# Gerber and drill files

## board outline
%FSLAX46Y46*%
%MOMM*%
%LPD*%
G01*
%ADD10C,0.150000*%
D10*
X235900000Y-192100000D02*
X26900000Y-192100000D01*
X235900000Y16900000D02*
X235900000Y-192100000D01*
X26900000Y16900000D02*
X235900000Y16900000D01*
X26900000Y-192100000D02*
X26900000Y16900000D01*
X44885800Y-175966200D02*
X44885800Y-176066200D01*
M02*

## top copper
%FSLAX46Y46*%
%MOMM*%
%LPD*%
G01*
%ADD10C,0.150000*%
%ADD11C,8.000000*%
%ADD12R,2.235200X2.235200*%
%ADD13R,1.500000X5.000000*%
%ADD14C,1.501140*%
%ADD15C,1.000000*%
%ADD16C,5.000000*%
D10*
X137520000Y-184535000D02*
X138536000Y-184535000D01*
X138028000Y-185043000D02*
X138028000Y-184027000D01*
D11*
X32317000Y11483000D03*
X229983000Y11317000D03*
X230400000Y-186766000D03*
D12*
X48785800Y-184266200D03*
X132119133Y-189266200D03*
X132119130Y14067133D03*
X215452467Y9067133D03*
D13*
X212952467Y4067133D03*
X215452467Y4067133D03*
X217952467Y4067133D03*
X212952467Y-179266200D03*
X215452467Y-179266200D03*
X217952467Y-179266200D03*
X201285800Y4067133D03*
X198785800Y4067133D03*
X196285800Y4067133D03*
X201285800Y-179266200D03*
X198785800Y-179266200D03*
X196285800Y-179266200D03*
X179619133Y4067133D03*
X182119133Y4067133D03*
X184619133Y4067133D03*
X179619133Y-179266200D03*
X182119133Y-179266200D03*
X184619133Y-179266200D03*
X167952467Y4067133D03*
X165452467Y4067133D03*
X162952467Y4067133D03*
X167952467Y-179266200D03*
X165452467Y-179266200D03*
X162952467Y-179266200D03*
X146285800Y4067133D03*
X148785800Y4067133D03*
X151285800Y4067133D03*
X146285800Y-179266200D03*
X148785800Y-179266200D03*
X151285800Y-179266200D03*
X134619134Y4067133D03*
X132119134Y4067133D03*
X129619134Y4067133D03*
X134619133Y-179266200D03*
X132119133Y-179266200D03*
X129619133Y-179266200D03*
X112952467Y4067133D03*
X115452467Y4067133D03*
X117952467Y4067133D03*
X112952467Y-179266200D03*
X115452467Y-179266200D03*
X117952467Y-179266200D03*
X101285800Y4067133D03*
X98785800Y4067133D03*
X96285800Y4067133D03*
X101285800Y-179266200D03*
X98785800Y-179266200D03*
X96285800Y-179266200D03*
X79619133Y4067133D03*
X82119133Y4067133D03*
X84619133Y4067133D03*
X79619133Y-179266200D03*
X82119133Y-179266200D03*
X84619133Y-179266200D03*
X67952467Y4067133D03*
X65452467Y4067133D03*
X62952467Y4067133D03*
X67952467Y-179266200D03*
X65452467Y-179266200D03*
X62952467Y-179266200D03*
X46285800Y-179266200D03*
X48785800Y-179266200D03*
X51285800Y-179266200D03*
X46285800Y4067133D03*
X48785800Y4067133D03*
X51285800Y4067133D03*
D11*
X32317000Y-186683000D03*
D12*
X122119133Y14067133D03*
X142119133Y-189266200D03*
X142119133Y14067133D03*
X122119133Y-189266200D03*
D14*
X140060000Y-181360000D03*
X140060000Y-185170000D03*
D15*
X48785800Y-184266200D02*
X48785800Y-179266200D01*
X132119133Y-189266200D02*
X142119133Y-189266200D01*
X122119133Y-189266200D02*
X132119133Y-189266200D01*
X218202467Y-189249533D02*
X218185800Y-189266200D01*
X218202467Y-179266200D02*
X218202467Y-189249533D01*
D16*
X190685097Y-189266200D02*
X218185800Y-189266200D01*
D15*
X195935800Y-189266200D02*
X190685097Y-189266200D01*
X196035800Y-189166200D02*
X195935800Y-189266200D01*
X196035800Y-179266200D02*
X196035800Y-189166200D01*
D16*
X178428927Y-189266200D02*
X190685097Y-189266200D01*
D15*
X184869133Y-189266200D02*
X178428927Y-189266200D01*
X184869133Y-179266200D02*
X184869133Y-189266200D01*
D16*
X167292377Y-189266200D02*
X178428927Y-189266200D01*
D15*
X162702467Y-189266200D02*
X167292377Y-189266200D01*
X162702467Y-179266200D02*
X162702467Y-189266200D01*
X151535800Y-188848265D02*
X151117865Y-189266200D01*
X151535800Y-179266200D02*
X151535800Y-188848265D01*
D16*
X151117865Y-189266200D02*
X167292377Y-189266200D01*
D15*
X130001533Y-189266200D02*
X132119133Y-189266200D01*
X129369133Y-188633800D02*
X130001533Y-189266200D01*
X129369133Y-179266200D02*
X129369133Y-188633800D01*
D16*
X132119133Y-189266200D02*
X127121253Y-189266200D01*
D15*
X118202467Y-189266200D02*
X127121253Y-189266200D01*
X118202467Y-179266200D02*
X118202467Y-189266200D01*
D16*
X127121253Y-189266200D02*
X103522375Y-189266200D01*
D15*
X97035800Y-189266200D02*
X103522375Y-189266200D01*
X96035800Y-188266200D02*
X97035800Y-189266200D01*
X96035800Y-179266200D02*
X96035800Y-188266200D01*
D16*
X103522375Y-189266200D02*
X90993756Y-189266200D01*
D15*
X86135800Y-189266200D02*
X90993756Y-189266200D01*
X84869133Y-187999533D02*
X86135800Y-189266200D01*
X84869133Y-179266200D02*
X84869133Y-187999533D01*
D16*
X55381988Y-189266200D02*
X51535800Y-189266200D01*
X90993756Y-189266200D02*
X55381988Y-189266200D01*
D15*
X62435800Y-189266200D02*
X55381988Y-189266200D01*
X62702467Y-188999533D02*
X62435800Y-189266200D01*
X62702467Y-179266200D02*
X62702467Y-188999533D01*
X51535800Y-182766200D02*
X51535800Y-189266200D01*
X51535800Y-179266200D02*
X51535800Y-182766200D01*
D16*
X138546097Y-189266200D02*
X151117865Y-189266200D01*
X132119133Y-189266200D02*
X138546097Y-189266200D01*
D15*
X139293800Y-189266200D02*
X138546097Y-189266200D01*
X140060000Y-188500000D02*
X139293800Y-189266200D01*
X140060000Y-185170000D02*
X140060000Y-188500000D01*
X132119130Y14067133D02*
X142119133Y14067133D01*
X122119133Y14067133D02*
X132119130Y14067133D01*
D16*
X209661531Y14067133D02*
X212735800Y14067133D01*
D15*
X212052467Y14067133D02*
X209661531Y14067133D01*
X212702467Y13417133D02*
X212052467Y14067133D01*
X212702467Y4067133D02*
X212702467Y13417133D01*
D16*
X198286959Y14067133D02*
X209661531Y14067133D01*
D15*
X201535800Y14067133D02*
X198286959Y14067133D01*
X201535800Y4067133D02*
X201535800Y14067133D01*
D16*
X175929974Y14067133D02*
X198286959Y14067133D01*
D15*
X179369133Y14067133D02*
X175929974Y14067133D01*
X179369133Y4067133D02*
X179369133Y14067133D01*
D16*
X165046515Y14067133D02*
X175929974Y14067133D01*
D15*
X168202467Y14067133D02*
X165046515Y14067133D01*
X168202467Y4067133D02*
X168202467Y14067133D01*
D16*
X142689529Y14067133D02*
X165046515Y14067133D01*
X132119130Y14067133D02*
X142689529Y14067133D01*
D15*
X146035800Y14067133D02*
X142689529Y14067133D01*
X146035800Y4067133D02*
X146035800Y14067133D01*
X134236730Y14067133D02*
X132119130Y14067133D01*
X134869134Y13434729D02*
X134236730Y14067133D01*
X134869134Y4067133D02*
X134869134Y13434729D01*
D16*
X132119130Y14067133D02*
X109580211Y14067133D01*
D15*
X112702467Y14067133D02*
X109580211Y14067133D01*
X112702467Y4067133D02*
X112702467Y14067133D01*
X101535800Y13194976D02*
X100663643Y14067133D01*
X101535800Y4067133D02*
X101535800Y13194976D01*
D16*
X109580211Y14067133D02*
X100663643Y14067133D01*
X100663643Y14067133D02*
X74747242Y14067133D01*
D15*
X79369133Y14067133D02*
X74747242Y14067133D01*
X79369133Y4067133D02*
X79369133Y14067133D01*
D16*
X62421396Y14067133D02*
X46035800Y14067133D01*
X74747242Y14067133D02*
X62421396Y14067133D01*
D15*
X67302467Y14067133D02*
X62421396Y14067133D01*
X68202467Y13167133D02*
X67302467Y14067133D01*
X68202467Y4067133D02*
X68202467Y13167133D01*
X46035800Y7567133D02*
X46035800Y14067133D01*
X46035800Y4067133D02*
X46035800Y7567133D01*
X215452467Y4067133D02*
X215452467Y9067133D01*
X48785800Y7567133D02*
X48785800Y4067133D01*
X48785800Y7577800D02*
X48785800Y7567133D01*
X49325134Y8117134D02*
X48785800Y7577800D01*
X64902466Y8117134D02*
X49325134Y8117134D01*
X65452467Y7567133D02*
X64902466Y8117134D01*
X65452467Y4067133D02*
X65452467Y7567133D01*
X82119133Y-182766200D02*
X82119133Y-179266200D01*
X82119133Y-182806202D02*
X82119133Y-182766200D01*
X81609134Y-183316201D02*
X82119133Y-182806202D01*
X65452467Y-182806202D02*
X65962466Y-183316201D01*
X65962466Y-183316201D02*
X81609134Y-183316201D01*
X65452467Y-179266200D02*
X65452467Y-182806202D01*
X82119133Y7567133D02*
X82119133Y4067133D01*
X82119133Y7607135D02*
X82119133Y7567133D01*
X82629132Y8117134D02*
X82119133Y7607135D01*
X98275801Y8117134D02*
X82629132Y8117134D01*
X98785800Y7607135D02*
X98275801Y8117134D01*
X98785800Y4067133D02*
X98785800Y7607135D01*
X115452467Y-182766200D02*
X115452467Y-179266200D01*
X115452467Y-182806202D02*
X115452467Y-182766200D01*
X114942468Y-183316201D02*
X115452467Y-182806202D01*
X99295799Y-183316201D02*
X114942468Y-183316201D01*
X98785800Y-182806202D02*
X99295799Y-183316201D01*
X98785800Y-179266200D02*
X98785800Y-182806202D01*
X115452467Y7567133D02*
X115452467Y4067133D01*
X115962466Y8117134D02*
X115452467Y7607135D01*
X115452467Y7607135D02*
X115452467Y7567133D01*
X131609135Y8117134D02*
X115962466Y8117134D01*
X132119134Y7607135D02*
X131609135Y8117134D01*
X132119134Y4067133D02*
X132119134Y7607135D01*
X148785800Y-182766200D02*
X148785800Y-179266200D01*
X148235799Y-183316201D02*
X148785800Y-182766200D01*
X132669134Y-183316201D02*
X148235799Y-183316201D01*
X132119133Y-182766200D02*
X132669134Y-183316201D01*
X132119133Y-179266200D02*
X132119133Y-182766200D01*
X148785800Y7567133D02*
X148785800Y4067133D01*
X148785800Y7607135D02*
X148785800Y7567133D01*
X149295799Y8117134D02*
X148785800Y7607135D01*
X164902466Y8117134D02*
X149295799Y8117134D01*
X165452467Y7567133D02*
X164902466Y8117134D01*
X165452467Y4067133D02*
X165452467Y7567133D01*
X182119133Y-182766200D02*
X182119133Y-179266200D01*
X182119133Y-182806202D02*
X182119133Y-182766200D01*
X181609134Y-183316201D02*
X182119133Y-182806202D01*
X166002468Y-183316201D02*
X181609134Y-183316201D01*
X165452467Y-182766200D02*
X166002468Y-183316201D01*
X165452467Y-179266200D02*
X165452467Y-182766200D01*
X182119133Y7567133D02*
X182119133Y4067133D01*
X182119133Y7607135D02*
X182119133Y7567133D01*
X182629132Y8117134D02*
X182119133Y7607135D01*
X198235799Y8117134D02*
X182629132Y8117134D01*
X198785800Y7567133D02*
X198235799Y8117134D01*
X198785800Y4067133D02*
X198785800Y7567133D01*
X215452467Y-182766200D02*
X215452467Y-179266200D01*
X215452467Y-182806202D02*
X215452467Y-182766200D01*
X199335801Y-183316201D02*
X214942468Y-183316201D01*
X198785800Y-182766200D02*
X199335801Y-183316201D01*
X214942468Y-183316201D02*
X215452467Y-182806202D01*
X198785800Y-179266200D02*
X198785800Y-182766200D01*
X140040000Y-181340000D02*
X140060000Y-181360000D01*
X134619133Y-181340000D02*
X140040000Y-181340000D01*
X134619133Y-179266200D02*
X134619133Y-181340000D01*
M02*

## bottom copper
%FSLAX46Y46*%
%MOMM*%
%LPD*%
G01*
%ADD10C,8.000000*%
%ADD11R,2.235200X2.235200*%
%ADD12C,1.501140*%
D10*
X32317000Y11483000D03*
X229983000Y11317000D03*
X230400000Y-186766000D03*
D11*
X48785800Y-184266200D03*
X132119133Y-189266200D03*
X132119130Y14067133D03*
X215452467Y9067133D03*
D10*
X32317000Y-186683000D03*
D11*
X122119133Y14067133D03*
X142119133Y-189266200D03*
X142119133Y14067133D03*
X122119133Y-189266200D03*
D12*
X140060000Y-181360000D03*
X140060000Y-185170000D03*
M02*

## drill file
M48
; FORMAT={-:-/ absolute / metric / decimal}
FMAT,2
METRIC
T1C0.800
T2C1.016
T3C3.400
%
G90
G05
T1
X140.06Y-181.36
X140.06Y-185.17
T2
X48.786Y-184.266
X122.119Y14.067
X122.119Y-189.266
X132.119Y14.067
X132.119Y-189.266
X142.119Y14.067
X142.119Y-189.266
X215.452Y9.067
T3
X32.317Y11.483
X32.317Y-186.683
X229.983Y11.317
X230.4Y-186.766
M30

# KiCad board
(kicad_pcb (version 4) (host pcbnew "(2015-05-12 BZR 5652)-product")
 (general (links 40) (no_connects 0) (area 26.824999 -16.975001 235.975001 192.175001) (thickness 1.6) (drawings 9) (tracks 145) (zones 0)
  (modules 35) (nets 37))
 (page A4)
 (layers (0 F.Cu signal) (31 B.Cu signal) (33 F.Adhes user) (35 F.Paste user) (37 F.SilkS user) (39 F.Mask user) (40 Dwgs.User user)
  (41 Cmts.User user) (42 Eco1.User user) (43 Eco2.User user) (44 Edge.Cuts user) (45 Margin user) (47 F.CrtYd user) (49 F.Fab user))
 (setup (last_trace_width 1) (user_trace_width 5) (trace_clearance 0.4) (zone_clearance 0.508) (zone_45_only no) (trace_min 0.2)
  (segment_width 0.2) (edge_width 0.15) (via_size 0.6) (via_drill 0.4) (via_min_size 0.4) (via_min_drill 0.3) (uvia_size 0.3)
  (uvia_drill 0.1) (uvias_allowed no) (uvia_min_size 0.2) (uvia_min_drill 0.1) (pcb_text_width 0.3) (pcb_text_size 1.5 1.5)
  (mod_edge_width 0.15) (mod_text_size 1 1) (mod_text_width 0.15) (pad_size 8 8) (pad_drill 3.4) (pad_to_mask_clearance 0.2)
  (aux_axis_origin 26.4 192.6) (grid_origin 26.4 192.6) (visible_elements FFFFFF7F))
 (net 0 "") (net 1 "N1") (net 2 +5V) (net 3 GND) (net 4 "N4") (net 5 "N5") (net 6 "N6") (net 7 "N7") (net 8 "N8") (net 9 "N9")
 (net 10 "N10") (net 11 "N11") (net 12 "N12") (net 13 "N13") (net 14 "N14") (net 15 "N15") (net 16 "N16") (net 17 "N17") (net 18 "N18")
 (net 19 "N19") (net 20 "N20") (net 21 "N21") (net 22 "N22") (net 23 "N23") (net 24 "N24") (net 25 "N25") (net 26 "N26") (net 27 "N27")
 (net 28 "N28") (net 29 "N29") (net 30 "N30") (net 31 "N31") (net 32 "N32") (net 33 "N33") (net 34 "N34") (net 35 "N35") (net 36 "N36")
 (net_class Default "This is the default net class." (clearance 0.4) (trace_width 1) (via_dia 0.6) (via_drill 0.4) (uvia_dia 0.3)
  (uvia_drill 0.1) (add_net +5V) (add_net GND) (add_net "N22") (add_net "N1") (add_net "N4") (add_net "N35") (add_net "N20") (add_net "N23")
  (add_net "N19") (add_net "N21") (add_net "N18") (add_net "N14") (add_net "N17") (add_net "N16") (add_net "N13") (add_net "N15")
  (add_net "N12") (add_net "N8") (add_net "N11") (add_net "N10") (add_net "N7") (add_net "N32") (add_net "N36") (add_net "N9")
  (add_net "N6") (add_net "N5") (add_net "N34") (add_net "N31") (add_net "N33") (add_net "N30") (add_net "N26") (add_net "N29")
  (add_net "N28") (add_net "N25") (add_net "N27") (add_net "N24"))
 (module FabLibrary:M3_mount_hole (layer F.Cu) (at 26.4 -17.4)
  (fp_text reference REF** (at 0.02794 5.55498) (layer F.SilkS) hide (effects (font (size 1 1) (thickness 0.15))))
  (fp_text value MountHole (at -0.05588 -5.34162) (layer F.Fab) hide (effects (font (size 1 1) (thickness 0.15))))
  (pad 1 thru_hole circle (at 5.917 5.917) (size 8 8) (drill 3.4) (layers *.Cu *.Mask F.SilkS)))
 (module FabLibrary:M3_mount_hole (layer F.Cu) (at 235.9 -17.234)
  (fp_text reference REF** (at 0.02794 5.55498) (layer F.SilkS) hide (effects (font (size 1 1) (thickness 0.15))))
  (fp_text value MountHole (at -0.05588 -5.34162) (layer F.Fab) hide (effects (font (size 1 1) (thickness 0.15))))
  (pad 1 thru_hole circle (at -5.917 5.917) (size 8 8) (drill 3.4) (layers *.Cu *.Mask F.SilkS)))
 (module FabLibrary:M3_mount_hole (layer F.Cu) (at 230.4 186.766)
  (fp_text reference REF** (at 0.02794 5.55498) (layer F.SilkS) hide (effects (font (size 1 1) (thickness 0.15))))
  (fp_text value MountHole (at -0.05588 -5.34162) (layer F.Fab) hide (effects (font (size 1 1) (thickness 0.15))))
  (pad 1 thru_hole circle (at 0 0) (size 8 8) (drill 3.4) (layers *.Cu *.Mask F.SilkS)))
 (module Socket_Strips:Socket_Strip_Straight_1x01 (layer F.Cu) (at 48.7858 184.2662 90)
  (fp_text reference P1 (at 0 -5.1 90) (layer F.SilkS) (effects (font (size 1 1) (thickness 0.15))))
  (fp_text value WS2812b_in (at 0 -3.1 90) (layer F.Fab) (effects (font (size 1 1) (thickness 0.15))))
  (pad 1 thru_hole rect (at 0 0 90) (size 2.2352 2.2352) (drill 1.016) (layers *.Cu *.Mask F.SilkS) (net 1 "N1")))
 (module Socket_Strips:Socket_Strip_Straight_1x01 (layer F.Cu) (at 132.119133 189.2662 90)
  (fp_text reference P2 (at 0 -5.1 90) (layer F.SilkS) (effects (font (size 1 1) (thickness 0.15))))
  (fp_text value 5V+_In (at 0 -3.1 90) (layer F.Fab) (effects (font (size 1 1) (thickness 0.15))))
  (pad 1 thru_hole rect (at 0 0 90) (size 2.2352 2.2352) (drill 1.016) (layers *.Cu *.Mask F.SilkS) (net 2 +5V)))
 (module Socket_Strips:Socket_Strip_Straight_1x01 (layer F.Cu) (at 132.11913 -14.067133 90)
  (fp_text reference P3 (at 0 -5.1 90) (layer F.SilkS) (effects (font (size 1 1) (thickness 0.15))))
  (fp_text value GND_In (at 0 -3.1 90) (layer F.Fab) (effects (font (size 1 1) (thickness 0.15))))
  (pad 1 thru_hole rect (at 0 0 90) (size 2.2352 2.2352) (drill 1.016) (layers *.Cu *.Mask F.SilkS) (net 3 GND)))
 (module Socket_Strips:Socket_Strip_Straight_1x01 (layer F.Cu) (at 215.452467 -9.067133 90)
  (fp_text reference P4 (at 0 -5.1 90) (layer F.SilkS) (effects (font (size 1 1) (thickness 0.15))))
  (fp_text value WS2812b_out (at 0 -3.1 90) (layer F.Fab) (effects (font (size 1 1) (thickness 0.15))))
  (pad 1 thru_hole rect (at 0 0 90) (size 2.2352 2.2352) (drill 1.016) (layers *.Cu *.Mask F.SilkS) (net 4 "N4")))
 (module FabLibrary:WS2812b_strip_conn (layer F.Cu) (at 215.452467 -4.067133 270)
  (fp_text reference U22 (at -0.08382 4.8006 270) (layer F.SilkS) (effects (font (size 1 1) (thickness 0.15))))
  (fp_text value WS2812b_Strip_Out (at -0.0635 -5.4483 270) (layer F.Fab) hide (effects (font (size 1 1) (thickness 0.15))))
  (pad 1 smd rect (at 0 2.5 270) (size 5 1.5) (layers F.Cu F.Paste F.Mask) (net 3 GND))
  (pad 2 smd rect (at 0 0 270) (size 5 1.5) (layers F.Cu F.Paste F.Mask) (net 4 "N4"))
  (pad 3 smd rect (at 0 -2.5 270) (size 5 1.5) (layers F.Cu F.Paste F.Mask) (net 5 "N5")))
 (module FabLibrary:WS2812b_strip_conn (layer F.Cu) (at 215.452467 179.2662 270)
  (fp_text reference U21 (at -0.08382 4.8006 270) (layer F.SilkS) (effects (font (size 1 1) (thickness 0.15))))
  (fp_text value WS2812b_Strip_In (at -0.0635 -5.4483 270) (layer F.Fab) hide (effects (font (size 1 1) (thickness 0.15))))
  (pad 1 smd rect (at 0 2.5 270) (size 5 1.5) (layers F.Cu F.Paste F.Mask) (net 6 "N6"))
  (pad 2 smd rect (at 0 0 270) (size 5 1.5) (layers F.Cu F.Paste F.Mask) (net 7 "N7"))
  (pad 3 smd rect (at 0 -2.5 270) (size 5 1.5) (layers F.Cu F.Paste F.Mask) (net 2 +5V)))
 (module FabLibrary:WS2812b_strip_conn (layer F.Cu) (at 198.7858 -4.067133 90)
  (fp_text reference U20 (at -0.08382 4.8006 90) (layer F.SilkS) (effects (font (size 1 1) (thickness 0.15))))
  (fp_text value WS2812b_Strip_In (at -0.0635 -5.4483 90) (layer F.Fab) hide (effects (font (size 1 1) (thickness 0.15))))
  (pad 1 smd rect (at 0 2.5 90) (size 5 1.5) (layers F.Cu F.Paste F.Mask) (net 3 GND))
  (pad 2 smd rect (at 0 0 90) (size 5 1.5) (layers F.Cu F.Paste F.Mask) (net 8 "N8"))
  (pad 3 smd rect (at 0 -2.5 90) (size 5 1.5) (layers F.Cu F.Paste F.Mask) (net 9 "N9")))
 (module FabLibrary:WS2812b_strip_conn (layer F.Cu) (at 198.7858 179.2662 90)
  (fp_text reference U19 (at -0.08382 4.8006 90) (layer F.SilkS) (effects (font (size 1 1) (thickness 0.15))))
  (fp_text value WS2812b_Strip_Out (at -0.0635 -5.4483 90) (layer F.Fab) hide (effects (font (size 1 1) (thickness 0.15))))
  (pad 1 smd rect (at 0 2.5 90) (size 5 1.5) (layers F.Cu F.Paste F.Mask) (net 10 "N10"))
  (pad 2 smd rect (at 0 0 90) (size 5 1.5) (layers F.Cu F.Paste F.Mask) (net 7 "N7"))
  (pad 3 smd rect (at 0 -2.5 90) (size 5 1.5) (layers F.Cu F.Paste F.Mask) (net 2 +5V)))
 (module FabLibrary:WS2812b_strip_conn (layer F.Cu) (at 182.119133 -4.067133 270)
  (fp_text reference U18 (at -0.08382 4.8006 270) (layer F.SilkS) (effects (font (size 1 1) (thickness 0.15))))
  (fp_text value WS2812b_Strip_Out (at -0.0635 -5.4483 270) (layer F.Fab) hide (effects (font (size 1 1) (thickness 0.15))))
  (pad 1 smd rect (at 0 2.5 270) (size 5 1.5) (layers F.Cu F.Paste F.Mask) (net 3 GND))
  (pad 2 smd rect (at 0 0 270) (size 5 1.5) (layers F.Cu F.Paste F.Mask) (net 8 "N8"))
  (pad 3 smd rect (at 0 -2.5 270) (size 5 1.5) (layers F.Cu F.Paste F.Mask) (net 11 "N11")))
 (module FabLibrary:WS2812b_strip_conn (layer F.Cu) (at 182.119133 179.2662 270)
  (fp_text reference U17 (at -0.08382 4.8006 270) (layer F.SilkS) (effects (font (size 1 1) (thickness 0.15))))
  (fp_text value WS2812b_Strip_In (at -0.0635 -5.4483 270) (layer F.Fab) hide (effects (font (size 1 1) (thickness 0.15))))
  (pad 1 smd rect (at 0 2.5 270) (size 5 1.5) (layers F.Cu F.Paste F.Mask) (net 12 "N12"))
  (pad 2 smd rect (at 0 0 270) (size 5 1.5) (layers F.Cu F.Paste F.Mask) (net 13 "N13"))
  (pad 3 smd rect (at 0 -2.5 270) (size 5 1.5) (layers F.Cu F.Paste F.Mask) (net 2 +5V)))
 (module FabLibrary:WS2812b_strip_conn (layer F.Cu) (at 165.452467 -4.067133 90)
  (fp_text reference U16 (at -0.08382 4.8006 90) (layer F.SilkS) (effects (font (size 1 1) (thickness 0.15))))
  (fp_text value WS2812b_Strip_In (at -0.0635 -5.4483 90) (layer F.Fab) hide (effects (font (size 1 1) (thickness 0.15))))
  (pad 1 smd rect (at 0 2.5 90) (size 5 1.5) (layers F.Cu F.Paste F.Mask) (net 3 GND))
  (pad 2 smd rect (at 0 0 90) (size 5 1.5) (layers F.Cu F.Paste F.Mask) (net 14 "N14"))
  (pad 3 smd rect (at 0 -2.5 90) (size 5 1.5) (layers F.Cu F.Paste F.Mask) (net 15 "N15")))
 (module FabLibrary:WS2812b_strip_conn (layer F.Cu) (at 165.452467 179.2662 90)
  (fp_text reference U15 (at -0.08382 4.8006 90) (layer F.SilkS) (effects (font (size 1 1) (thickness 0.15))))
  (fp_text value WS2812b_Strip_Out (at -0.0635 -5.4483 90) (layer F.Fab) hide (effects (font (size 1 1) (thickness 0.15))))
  (pad 1 smd rect (at 0 2.5 90) (size 5 1.5) (layers F.Cu F.Paste F.Mask) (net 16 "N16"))
  (pad 2 smd rect (at 0 0 90) (size 5 1.5) (layers F.Cu F.Paste F.Mask) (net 13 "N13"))
  (pad 3 smd rect (at 0 -2.5 90) (size 5 1.5) (layers F.Cu F.Paste F.Mask) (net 2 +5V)))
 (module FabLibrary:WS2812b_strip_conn (layer F.Cu) (at 148.7858 -4.067133 270)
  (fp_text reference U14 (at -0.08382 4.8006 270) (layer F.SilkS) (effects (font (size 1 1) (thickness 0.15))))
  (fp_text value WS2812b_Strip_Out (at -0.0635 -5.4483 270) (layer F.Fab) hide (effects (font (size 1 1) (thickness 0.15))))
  (pad 1 smd rect (at 0 2.5 270) (size 5 1.5) (layers F.Cu F.Paste F.Mask) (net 3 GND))
  (pad 2 smd rect (at 0 0 270) (size 5 1.5) (layers F.Cu F.Paste F.Mask) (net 14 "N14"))
  (pad 3 smd rect (at 0 -2.5 270) (size 5 1.5) (layers F.Cu F.Paste F.Mask) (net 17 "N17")))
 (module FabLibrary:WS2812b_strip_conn (layer F.Cu) (at 148.7858 179.2662 270)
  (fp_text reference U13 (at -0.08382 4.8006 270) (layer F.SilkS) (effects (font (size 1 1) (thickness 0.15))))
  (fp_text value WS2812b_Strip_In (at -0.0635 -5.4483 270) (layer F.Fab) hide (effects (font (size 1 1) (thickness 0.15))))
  (pad 1 smd rect (at 0 2.5 270) (size 5 1.5) (layers F.Cu F.Paste F.Mask) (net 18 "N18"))
  (pad 2 smd rect (at 0 0 270) (size 5 1.5) (layers F.Cu F.Paste F.Mask) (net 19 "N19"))
  (pad 3 smd rect (at 0 -2.5 270) (size 5 1.5) (layers F.Cu F.Paste F.Mask) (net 2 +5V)))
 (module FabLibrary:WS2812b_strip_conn (layer F.Cu) (at 132.119134 -4.067133 90)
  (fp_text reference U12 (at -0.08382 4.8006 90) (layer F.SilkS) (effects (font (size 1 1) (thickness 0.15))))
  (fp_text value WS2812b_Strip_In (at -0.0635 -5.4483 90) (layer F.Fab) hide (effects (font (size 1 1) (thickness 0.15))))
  (pad 1 smd rect (at 0 2.5 90) (size 5 1.5) (layers F.Cu F.Paste F.Mask) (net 3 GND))
  (pad 2 smd rect (at 0 0 90) (size 5 1.5) (layers F.Cu F.Paste F.Mask) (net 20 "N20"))
  (pad 3 smd rect (at 0 -2.5 90) (size 5 1.5) (layers F.Cu F.Paste F.Mask) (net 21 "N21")))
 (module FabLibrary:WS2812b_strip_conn (layer F.Cu) (at 132.119133 179.2662 90)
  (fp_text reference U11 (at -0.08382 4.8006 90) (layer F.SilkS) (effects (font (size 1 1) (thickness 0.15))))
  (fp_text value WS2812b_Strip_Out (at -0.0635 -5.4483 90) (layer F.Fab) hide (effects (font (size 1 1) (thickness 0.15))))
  (pad 1 smd rect (at 0 2.5 90) (size 5 1.5) (layers F.Cu F.Paste F.Mask) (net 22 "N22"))
  (pad 2 smd rect (at 0 0 90) (size 5 1.5) (layers F.Cu F.Paste F.Mask) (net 19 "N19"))
  (pad 3 smd rect (at 0 -2.5 90) (size 5 1.5) (layers F.Cu F.Paste F.Mask) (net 2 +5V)))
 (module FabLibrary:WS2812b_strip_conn (layer F.Cu) (at 115.452467 -4.067133 270)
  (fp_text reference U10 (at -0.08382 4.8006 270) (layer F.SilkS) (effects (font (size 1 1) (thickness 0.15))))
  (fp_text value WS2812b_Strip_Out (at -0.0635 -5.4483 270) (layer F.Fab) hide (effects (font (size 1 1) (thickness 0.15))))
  (pad 1 smd rect (at 0 2.5 270) (size 5 1.5) (layers F.Cu F.Paste F.Mask) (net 3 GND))
  (pad 2 smd rect (at 0 0 270) (size 5 1.5) (layers F.Cu F.Paste F.Mask) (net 20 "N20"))
  (pad 3 smd rect (at 0 -2.5 270) (size 5 1.5) (layers F.Cu F.Paste F.Mask) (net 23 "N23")))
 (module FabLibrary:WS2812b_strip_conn (layer F.Cu) (at 115.452467 179.2662 270)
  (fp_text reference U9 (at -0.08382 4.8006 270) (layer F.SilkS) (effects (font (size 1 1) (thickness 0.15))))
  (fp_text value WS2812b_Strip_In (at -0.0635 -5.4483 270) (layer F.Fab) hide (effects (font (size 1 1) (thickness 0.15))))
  (pad 1 smd rect (at 0 2.5 270) (size 5 1.5) (layers F.Cu F.Paste F.Mask) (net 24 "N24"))
  (pad 2 smd rect (at 0 0 270) (size 5 1.5) (layers F.Cu F.Paste F.Mask) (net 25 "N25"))
  (pad 3 smd rect (at 0 -2.5 270) (size 5 1.5) (layers F.Cu F.Paste F.Mask) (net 2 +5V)))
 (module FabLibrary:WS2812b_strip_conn (layer F.Cu) (at 98.7858 -4.067133 90)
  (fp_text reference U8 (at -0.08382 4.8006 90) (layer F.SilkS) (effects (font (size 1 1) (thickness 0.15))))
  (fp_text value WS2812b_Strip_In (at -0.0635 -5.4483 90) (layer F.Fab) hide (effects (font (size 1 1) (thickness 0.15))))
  (pad 1 smd rect (at 0 2.5 90) (size 5 1.5) (layers F.Cu F.Paste F.Mask) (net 3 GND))
  (pad 2 smd rect (at 0 0 90) (size 5 1.5) (layers F.Cu F.Paste F.Mask) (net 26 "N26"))
  (pad 3 smd rect (at 0 -2.5 90) (size 5 1.5) (layers F.Cu F.Paste F.Mask) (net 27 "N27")))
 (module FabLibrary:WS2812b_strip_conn (layer F.Cu) (at 98.7858 179.2662 90)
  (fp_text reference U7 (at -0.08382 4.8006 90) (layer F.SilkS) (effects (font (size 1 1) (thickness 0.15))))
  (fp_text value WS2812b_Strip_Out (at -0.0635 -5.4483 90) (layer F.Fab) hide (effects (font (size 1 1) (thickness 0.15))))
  (pad 1 smd rect (at 0 2.5 90) (size 5 1.5) (layers F.Cu F.Paste F.Mask) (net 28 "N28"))
  (pad 2 smd rect (at 0 0 90) (size 5 1.5) (layers F.Cu F.Paste F.Mask) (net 25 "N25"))
  (pad 3 smd rect (at 0 -2.5 90) (size 5 1.5) (layers F.Cu F.Paste F.Mask) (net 2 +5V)))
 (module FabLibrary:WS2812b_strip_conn (layer F.Cu) (at 82.119133 -4.067133 270)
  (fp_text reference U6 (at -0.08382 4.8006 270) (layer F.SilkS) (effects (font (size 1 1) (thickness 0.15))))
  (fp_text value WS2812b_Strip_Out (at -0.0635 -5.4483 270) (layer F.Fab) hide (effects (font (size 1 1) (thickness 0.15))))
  (pad 1 smd rect (at 0 2.5 270) (size 5 1.5) (layers F.Cu F.Paste F.Mask) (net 3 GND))
  (pad 2 smd rect (at 0 0 270) (size 5 1.5) (layers F.Cu F.Paste F.Mask) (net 26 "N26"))
  (pad 3 smd rect (at 0 -2.5 270) (size 5 1.5) (layers F.Cu F.Paste F.Mask) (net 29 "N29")))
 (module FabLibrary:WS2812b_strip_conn (layer F.Cu) (at 82.119133 179.2662 270)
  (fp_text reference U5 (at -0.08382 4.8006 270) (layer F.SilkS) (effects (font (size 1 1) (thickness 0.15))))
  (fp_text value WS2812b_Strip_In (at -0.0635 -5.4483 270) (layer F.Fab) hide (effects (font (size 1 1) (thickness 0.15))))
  (pad 1 smd rect (at 0 2.5 270) (size 5 1.5) (layers F.Cu F.Paste F.Mask) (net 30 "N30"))
  (pad 2 smd rect (at 0 0 270) (size 5 1.5) (layers F.Cu F.Paste F.Mask) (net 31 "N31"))
  (pad 3 smd rect (at 0 -2.5 270) (size 5 1.5) (layers F.Cu F.Paste F.Mask) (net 2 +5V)))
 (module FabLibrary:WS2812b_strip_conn (layer F.Cu) (at 65.452467 -4.067133 90)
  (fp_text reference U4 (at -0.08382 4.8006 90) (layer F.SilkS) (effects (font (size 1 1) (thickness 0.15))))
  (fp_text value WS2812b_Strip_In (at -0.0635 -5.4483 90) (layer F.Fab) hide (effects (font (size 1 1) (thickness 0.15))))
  (pad 1 smd rect (at 0 2.5 90) (size 5 1.5) (layers F.Cu F.Paste F.Mask) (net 3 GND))
  (pad 2 smd rect (at 0 0 90) (size 5 1.5) (layers F.Cu F.Paste F.Mask) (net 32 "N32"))
  (pad 3 smd rect (at 0 -2.5 90) (size 5 1.5) (layers F.Cu F.Paste F.Mask) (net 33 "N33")))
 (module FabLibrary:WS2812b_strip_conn (layer F.Cu) (at 65.452467 179.2662 90)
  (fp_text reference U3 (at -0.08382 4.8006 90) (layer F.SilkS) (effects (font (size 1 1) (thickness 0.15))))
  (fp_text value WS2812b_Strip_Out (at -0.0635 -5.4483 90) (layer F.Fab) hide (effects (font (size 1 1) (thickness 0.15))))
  (pad 1 smd rect (at 0 2.5 90) (size 5 1.5) (layers F.Cu F.Paste F.Mask) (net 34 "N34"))
  (pad 2 smd rect (at 0 0 90) (size 5 1.5) (layers F.Cu F.Paste F.Mask) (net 31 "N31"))
  (pad 3 smd rect (at 0 -2.5 90) (size 5 1.5) (layers F.Cu F.Paste F.Mask) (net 2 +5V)))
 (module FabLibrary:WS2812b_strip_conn (layer F.Cu) (at 48.7858 179.2662 270)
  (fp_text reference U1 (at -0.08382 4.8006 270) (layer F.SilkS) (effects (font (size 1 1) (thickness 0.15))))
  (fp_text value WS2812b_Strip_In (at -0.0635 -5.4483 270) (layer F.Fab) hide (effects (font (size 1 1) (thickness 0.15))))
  (pad 1 smd rect (at 0 2.5 270) (size 5 1.5) (layers F.Cu F.Paste F.Mask) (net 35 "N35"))
  (pad 2 smd rect (at 0 0 270) (size 5 1.5) (layers F.Cu F.Paste F.Mask) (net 1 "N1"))
  (pad 3 smd rect (at 0 -2.5 270) (size 5 1.5) (layers F.Cu F.Paste F.Mask) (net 2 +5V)))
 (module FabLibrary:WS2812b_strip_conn (layer F.Cu) (at 48.7858 -4.067133 270)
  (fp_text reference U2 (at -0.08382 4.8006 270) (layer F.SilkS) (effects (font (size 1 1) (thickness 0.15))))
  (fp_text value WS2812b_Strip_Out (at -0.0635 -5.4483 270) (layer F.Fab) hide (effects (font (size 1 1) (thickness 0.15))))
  (pad 1 smd rect (at 0 2.5 270) (size 5 1.5) (layers F.Cu F.Paste F.Mask) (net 3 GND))
  (pad 2 smd rect (at 0 0 270) (size 5 1.5) (layers F.Cu F.Paste F.Mask) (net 32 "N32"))
  (pad 3 smd rect (at 0 -2.5 270) (size 5 1.5) (layers F.Cu F.Paste F.Mask) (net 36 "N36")))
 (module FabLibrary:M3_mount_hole (layer F.Cu) (at 32.317 186.683)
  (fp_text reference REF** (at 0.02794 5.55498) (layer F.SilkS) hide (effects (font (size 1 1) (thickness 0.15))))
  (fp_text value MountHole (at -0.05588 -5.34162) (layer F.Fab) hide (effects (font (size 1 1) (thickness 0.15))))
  (pad 1 thru_hole circle (at 0 0) (size 8 8) (drill 3.4) (layers *.Cu *.Mask F.SilkS)))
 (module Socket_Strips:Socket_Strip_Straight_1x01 (layer F.Cu) (at 122.119133 -14.067133)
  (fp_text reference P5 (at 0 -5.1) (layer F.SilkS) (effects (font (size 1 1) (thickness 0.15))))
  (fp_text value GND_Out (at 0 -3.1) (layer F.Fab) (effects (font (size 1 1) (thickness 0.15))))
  (pad 1 thru_hole rect (at 0 0) (size 2.2352 2.2352) (drill 1.016) (layers *.Cu *.Mask F.SilkS) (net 3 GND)))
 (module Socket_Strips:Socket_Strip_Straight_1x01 (layer F.Cu) (at 142.119133 189.2662)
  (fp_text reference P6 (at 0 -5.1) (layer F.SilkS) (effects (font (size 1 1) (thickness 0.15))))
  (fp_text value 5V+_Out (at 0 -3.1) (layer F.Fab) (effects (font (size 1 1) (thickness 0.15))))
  (pad 1 thru_hole rect (at 0 0) (size 2.2352 2.2352) (drill 1.016) (layers *.Cu *.Mask F.SilkS) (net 2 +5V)))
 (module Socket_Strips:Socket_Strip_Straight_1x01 (layer F.Cu) (at 142.119133 -14.067133)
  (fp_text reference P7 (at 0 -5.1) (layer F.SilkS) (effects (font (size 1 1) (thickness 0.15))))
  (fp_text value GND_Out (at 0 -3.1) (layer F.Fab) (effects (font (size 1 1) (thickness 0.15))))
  (pad 1 thru_hole rect (at 0 0) (size 2.2352 2.2352) (drill 1.016) (layers *.Cu *.Mask F.SilkS) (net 3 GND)))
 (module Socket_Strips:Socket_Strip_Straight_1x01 (layer F.Cu) (at 122.119133 189.2662)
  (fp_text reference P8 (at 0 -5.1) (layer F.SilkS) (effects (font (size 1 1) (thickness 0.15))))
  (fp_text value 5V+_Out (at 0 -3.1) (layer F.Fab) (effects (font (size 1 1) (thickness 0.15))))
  (pad 1 thru_hole rect (at 0 0) (size 2.2352 2.2352) (drill 1.016) (layers *.Cu *.Mask F.SilkS) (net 2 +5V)))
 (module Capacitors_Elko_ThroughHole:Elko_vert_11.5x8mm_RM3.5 (layer F.Cu) (at 140.06 185.17 90)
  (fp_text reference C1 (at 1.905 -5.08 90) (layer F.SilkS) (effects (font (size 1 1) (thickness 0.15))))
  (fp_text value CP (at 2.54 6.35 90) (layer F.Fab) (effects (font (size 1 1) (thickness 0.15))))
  (fp_line (start 0.635 -2.54) (end 0.635 -1.524) (layer F.Cu) (width 0.15))
  (fp_line (start 0.127 -2.032) (end 1.143 -2.032) (layer F.Cu) (width 0.15))
  (pad 2 thru_hole circle (at 3.81 0 90) (size 1.50114 1.50114) (drill 0.8001) (layers *.Cu *.Mask F.SilkS) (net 22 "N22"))
  (pad 1 thru_hole circle (at 0 0 90) (size 1.50114 1.50114) (drill 0.8001) (layers *.Cu *.Mask F.SilkS) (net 2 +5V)))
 (gr_line (start 235.9 192.1) (end 26.9 192.1) (angle 90) (layer Edge.Cuts) (width 0.15))
 (gr_line (start 235.9 -16.9) (end 235.9 192.1) (angle 90) (layer Edge.Cuts) (width 0.15))
 (gr_line (start 26.9 -16.9) (end 235.9 -16.9) (angle 90) (layer Edge.Cuts) (width 0.15))
 (gr_line (start 26.9 192.1) (end 26.9 -16.9) (angle 90) (layer Edge.Cuts) (width 0.15))
 (gr_line (start 44.8858 175.9662) (end 44.8858 176.0662) (angle 90) (layer Edge.Cuts) (width 0.15))
 (segment (start 48.7858 184.2662) (end 48.7858 179.2662) (width 1) (layer F.Cu) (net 1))
 (segment (start 132.119133 189.2662) (end 142.119133 189.2662) (width 1) (layer F.Cu) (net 2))
 (segment (start 122.119133 189.2662) (end 132.119133 189.2662) (width 1) (layer F.Cu) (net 2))
 (segment (start 218.202467 189.249533) (end 218.1858 189.2662) (width 1) (layer F.Cu) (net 2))
 (segment (start 218.202467 179.2662) (end 218.202467 189.249533) (width 1) (layer F.Cu) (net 2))
 (segment (start 190.685097 189.2662) (end 218.1858 189.2662) (width 5) (layer F.Cu) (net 2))
 (segment (start 195.9358 189.2662) (end 190.685097 189.2662) (width 1) (layer F.Cu) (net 2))
 (segment (start 196.0358 189.1662) (end 195.9358 189.2662) (width 1) (layer F.Cu) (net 2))
 (segment (start 196.0358 179.2662) (end 196.0358 189.1662) (width 1) (layer F.Cu) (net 2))
 (segment (start 178.428927 189.2662) (end 190.685097 189.2662) (width 5) (layer F.Cu) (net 2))
 (segment (start 184.869133 189.2662) (end 178.428927 189.2662) (width 1) (layer F.Cu) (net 2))
 (segment (start 184.869133 179.2662) (end 184.869133 189.2662) (width 1) (layer F.Cu) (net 2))
 (segment (start 167.292377 189.2662) (end 178.428927 189.2662) (width 5) (layer F.Cu) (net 2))
 (segment (start 162.702467 189.2662) (end 167.292377 189.2662) (width 1) (layer F.Cu) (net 2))
 (segment (start 162.702467 179.2662) (end 162.702467 189.2662) (width 1) (layer F.Cu) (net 2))
 (segment (start 151.5358 188.848265) (end 151.117865 189.2662) (width 1) (layer F.Cu) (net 2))
 (segment (start 151.5358 179.2662) (end 151.5358 188.848265) (width 1) (layer F.Cu) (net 2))
 (segment (start 151.117865 189.2662) (end 167.292377 189.2662) (width 5) (layer F.Cu) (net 2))
 (segment (start 130.001533 189.2662) (end 132.119133 189.2662) (width 1) (layer F.Cu) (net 2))
 (segment (start 129.369133 188.6338) (end 130.001533 189.2662) (width 1) (layer F.Cu) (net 2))
 (segment (start 129.369133 179.2662) (end 129.369133 188.6338) (width 1) (layer F.Cu) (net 2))
 (segment (start 132.119133 189.2662) (end 127.121253 189.2662) (width 5) (layer F.Cu) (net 2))
 (segment (start 118.202467 189.2662) (end 127.121253 189.2662) (width 1) (layer F.Cu) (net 2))
 (segment (start 118.202467 179.2662) (end 118.202467 189.2662) (width 1) (layer F.Cu) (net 2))
 (segment (start 127.121253 189.2662) (end 103.522375 189.2662) (width 5) (layer F.Cu) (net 2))
 (segment (start 97.0358 189.2662) (end 103.522375 189.2662) (width 1) (layer F.Cu) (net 2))
 (segment (start 96.0358 188.2662) (end 97.0358 189.2662) (width 1) (layer F.Cu) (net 2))
 (segment (start 96.0358 179.2662) (end 96.0358 188.2662) (width 1) (layer F.Cu) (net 2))
 (segment (start 103.522375 189.2662) (end 90.993756 189.2662) (width 5) (layer F.Cu) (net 2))
 (segment (start 86.1358 189.2662) (end 90.993756 189.2662) (width 1) (layer F.Cu) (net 2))
 (segment (start 84.869133 187.999533) (end 86.1358 189.2662) (width 1) (layer F.Cu) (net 2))
 (segment (start 84.869133 179.2662) (end 84.869133 187.999533) (width 1) (layer F.Cu) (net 2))
 (segment (start 55.381988 189.2662) (end 51.5358 189.2662) (width 5) (layer F.Cu) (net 2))
 (segment (start 90.993756 189.2662) (end 55.381988 189.2662) (width 5) (layer F.Cu) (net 2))
 (segment (start 62.4358 189.2662) (end 55.381988 189.2662) (width 1) (layer F.Cu) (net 2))
 (segment (start 62.702467 188.999533) (end 62.4358 189.2662) (width 1) (layer F.Cu) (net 2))
 (segment (start 62.702467 179.2662) (end 62.702467 188.999533) (width 1) (layer F.Cu) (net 2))
 (segment (start 51.5358 182.7662) (end 51.5358 189.2662) (width 1) (layer F.Cu) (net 2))
 (segment (start 51.5358 179.2662) (end 51.5358 182.7662) (width 1) (layer F.Cu) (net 2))
 (segment (start 138.546097 189.2662) (end 151.117865 189.2662) (width 5) (layer F.Cu) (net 2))
 (segment (start 132.119133 189.2662) (end 138.546097 189.2662) (width 5) (layer F.Cu) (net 2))
 (segment (start 139.2938 189.2662) (end 138.546097 189.2662) (width 1) (layer F.Cu) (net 2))
 (segment (start 140.06 188.5) (end 139.2938 189.2662) (width 1) (layer F.Cu) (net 2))
 (segment (start 140.06 185.17) (end 140.06 188.5) (width 1) (layer F.Cu) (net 2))
 (segment (start 132.11913 -14.067133) (end 142.119133 -14.067133) (width 1) (layer F.Cu) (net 3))
 (segment (start 122.119133 -14.067133) (end 132.11913 -14.067133) (width 1) (layer F.Cu) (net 3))
 (segment (start 209.661531 -14.067133) (end 212.7358 -14.067133) (width 5) (layer F.Cu) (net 3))
 (segment (start 212.052467 -14.067133) (end 209.661531 -14.067133) (width 1) (layer F.Cu) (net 3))
 (segment (start 212.702467 -13.417133) (end 212.052467 -14.067133) (width 1) (layer F.Cu) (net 3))
 (segment (start 212.702467 -4.067133) (end 212.702467 -13.417133) (width 1) (layer F.Cu) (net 3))
 (segment (start 198.286959 -14.067133) (end 209.661531 -14.067133) (width 5) (layer F.Cu) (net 3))
 (segment (start 201.5358 -14.067133) (end 198.286959 -14.067133) (width 1) (layer F.Cu) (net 3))
 (segment (start 201.5358 -4.067133) (end 201.5358 -14.067133) (width 1) (layer F.Cu) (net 3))
 (segment (start 175.929974 -14.067133) (end 198.286959 -14.067133) (width 5) (layer F.Cu) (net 3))
 (segment (start 179.369133 -14.067133) (end 175.929974 -14.067133) (width 1) (layer F.Cu) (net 3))
 (segment (start 179.369133 -4.067133) (end 179.369133 -14.067133) (width 1) (layer F.Cu) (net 3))
 (segment (start 165.046515 -14.067133) (end 175.929974 -14.067133) (width 5) (layer F.Cu) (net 3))
 (segment (start 168.202467 -14.067133) (end 165.046515 -14.067133) (width 1) (layer F.Cu) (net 3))
 (segment (start 168.202467 -4.067133) (end 168.202467 -14.067133) (width 1) (layer F.Cu) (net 3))
 (segment (start 142.689529 -14.067133) (end 165.046515 -14.067133) (width 5) (layer F.Cu) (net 3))
 (segment (start 132.11913 -14.067133) (end 142.689529 -14.067133) (width 5) (layer F.Cu) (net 3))
 (segment (start 146.0358 -14.067133) (end 142.689529 -14.067133) (width 1) (layer F.Cu) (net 3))
 (segment (start 146.0358 -4.067133) (end 146.0358 -14.067133) (width 1) (layer F.Cu) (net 3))
 (segment (start 134.23673 -14.067133) (end 132.11913 -14.067133) (width 1) (layer F.Cu) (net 3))
 (segment (start 134.869134 -13.434729) (end 134.23673 -14.067133) (width 1) (layer F.Cu) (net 3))
 (segment (start 134.869134 -4.067133) (end 134.869134 -13.434729) (width 1) (layer F.Cu) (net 3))
 (segment (start 132.11913 -14.067133) (end 109.580211 -14.067133) (width 5) (layer F.Cu) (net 3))
 (segment (start 112.702467 -14.067133) (end 109.580211 -14.067133) (width 1) (layer F.Cu) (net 3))
 (segment (start 112.702467 -4.067133) (end 112.702467 -14.067133) (width 1) (layer F.Cu) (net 3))
 (segment (start 101.5358 -13.194976) (end 100.663643 -14.067133) (width 1) (layer F.Cu) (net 3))
 (segment (start 101.5358 -4.067133) (end 101.5358 -13.194976) (width 1) (layer F.Cu) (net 3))
 (segment (start 109.580211 -14.067133) (end 100.663643 -14.067133) (width 5) (layer F.Cu) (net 3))
 (segment (start 100.663643 -14.067133) (end 74.747242 -14.067133) (width 5) (layer F.Cu) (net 3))
 (segment (start 79.369133 -14.067133) (end 74.747242 -14.067133) (width 1) (layer F.Cu) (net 3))
 (segment (start 79.369133 -4.067133) (end 79.369133 -14.067133) (width 1) (layer F.Cu) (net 3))
 (segment (start 62.421396 -14.067133) (end 46.0358 -14.067133) (width 5) (layer F.Cu) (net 3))
 (segment (start 74.747242 -14.067133) (end 62.421396 -14.067133) (width 5) (layer F.Cu) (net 3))
 (segment (start 67.302467 -14.067133) (end 62.421396 -14.067133) (width 1) (layer F.Cu) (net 3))
 (segment (start 68.202467 -13.167133) (end 67.302467 -14.067133) (width 1) (layer F.Cu) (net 3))
 (segment (start 68.202467 -4.067133) (end 68.202467 -13.167133) (width 1) (layer F.Cu) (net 3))
 (segment (start 46.0358 -7.567133) (end 46.0358 -14.067133) (width 1) (layer F.Cu) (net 3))
 (segment (start 46.0358 -4.067133) (end 46.0358 -7.567133) (width 1) (layer F.Cu) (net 3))
 (segment (start 215.452467 -4.067133) (end 215.452467 -9.067133) (width 1) (layer F.Cu) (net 4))
 (segment (start 48.7858 -7.567133) (end 48.7858 -4.067133) (width 1) (layer F.Cu) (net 32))
 (segment (start 48.7858 -7.5778) (end 48.7858 -7.567133) (width 1) (layer F.Cu) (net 32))
 (segment (start 49.325134 -8.117134) (end 48.7858 -7.5778) (width 1) (layer F.Cu) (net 32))
 (segment (start 64.902466 -8.117134) (end 49.325134 -8.117134) (width 1) (layer F.Cu) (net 32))
 (segment (start 65.452467 -7.567133) (end 64.902466 -8.117134) (width 1) (layer F.Cu) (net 32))
 (segment (start 65.452467 -4.067133) (end 65.452467 -7.567133) (width 1) (layer F.Cu) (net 32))
 (segment (start 82.119133 182.7662) (end 82.119133 179.2662) (width 1) (layer F.Cu) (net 31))
 (segment (start 82.119133 182.806202) (end 82.119133 182.7662) (width 1) (layer F.Cu) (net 31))
 (segment (start 81.609134 183.316201) (end 82.119133 182.806202) (width 1) (layer F.Cu) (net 31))
 (segment (start 65.452467 182.806202) (end 65.962466 183.316201) (width 1) (layer F.Cu) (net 31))
 (segment (start 65.962466 183.316201) (end 81.609134 183.316201) (width 1) (layer F.Cu) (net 31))
 (segment (start 65.452467 179.2662) (end 65.452467 182.806202) (width 1) (layer F.Cu) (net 31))
 (segment (start 82.119133 -7.567133) (end 82.119133 -4.067133) (width 1) (layer F.Cu) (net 26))
 (segment (start 82.119133 -7.607135) (end 82.119133 -7.567133) (width 1) (layer F.Cu) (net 26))
 (segment (start 82.629132 -8.117134) (end 82.119133 -7.607135) (width 1) (layer F.Cu) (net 26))
 (segment (start 98.275801 -8.117134) (end 82.629132 -8.117134) (width 1) (layer F.Cu) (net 26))
 (segment (start 98.7858 -7.607135) (end 98.275801 -8.117134) (width 1) (layer F.Cu) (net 26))
 (segment (start 98.7858 -4.067133) (end 98.7858 -7.607135) (width 1) (layer F.Cu) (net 26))
 (segment (start 115.452467 182.7662) (end 115.452467 179.2662) (width 1) (layer F.Cu) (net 25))
 (segment (start 115.452467 182.806202) (end 115.452467 182.7662) (width 1) (layer F.Cu) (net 25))
 (segment (start 114.942468 183.316201) (end 115.452467 182.806202) (width 1) (layer F.Cu) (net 25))
 (segment (start 99.295799 183.316201) (end 114.942468 183.316201) (width 1) (layer F.Cu) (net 25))
 (segment (start 98.7858 182.806202) (end 99.295799 183.316201) (width 1) (layer F.Cu) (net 25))
 (segment (start 98.7858 179.2662) (end 98.7858 182.806202) (width 1) (layer F.Cu) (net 25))
 (segment (start 115.452467 -7.567133) (end 115.452467 -4.067133) (width 1) (layer F.Cu) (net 20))
 (segment (start 115.962466 -8.117134) (end 115.452467 -7.607135) (width 1) (layer F.Cu) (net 20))
 (segment (start 115.452467 -7.607135) (end 115.452467 -7.567133) (width 1) (layer F.Cu) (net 20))
 (segment (start 131.609135 -8.117134) (end 115.962466 -8.117134) (width 1) (layer F.Cu) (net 20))
 (segment (start 132.119134 -7.607135) (end 131.609135 -8.117134) (width 1) (layer F.Cu) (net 20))
 (segment (start 132.119134 -4.067133) (end 132.119134 -7.607135) (width 1) (layer F.Cu) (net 20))
 (segment (start 148.7858 182.7662) (end 148.7858 179.2662) (width 1) (layer F.Cu) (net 19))
 (segment (start 148.235799 183.316201) (end 148.7858 182.7662) (width 1) (layer F.Cu) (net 19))
 (segment (start 132.669134 183.316201) (end 148.235799 183.316201) (width 1) (layer F.Cu) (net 19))
 (segment (start 132.119133 182.7662) (end 132.669134 183.316201) (width 1) (layer F.Cu) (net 19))
 (segment (start 132.119133 179.2662) (end 132.119133 182.7662) (width 1) (layer F.Cu) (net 19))
 (segment (start 148.7858 -7.567133) (end 148.7858 -4.067133) (width 1) (layer F.Cu) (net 14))
 (segment (start 148.7858 -7.607135) (end 148.7858 -7.567133) (width 1) (layer F.Cu) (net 14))
 (segment (start 149.295799 -8.117134) (end 148.7858 -7.607135) (width 1) (layer F.Cu) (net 14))
 (segment (start 164.902466 -8.117134) (end 149.295799 -8.117134) (width 1) (layer F.Cu) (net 14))
 (segment (start 165.452467 -7.567133) (end 164.902466 -8.117134) (width 1) (layer F.Cu) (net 14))
 (segment (start 165.452467 -4.067133) (end 165.452467 -7.567133) (width 1) (layer F.Cu) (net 14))
 (segment (start 182.119133 182.7662) (end 182.119133 179.2662) (width 1) (layer F.Cu) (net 13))
 (segment (start 182.119133 182.806202) (end 182.119133 182.7662) (width 1) (layer F.Cu) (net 13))
 (segment (start 181.609134 183.316201) (end 182.119133 182.806202) (width 1) (layer F.Cu) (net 13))
 (segment (start 166.002468 183.316201) (end 181.609134 183.316201) (width 1) (layer F.Cu) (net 13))
 (segment (start 165.452467 182.7662) (end 166.002468 183.316201) (width 1) (layer F.Cu) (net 13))
 (segment (start 165.452467 179.2662) (end 165.452467 182.7662) (width 1) (layer F.Cu) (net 13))
 (segment (start 182.119133 -7.567133) (end 182.119133 -4.067133) (width 1) (layer F.Cu) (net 8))
 (segment (start 182.119133 -7.607135) (end 182.119133 -7.567133) (width 1) (layer F.Cu) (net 8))
 (segment (start 182.629132 -8.117134) (end 182.119133 -7.607135) (width 1) (layer F.Cu) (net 8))
 (segment (start 198.235799 -8.117134) (end 182.629132 -8.117134) (width 1) (layer F.Cu) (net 8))
 (segment (start 198.7858 -7.567133) (end 198.235799 -8.117134) (width 1) (layer F.Cu) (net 8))
 (segment (start 198.7858 -4.067133) (end 198.7858 -7.567133) (width 1) (layer F.Cu) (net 8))
 (segment (start 215.452467 182.7662) (end 215.452467 179.2662) (width 1) (layer F.Cu) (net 7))
 (segment (start 215.452467 182.806202) (end 215.452467 182.7662) (width 1) (layer F.Cu) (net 7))
 (segment (start 199.335801 183.316201) (end 214.942468 183.316201) (width 1) (layer F.Cu) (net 7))
 (segment (start 198.7858 182.7662) (end 199.335801 183.316201) (width 1) (layer F.Cu) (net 7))
 (segment (start 214.942468 183.316201) (end 215.452467 182.806202) (width 1) (layer F.Cu) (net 7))
 (segment (start 198.7858 179.2662) (end 198.7858 182.7662) (width 1) (layer F.Cu) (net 7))
 (segment (start 140.04 181.34) (end 140.06 181.36) (width 1) (layer F.Cu) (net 22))
 (segment (start 134.619133 181.34) (end 140.04 181.34) (width 1) (layer F.Cu) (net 22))
 (segment (start 134.619133 179.2662) (end 134.619133 181.34) (width 1) (layer F.Cu) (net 22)))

